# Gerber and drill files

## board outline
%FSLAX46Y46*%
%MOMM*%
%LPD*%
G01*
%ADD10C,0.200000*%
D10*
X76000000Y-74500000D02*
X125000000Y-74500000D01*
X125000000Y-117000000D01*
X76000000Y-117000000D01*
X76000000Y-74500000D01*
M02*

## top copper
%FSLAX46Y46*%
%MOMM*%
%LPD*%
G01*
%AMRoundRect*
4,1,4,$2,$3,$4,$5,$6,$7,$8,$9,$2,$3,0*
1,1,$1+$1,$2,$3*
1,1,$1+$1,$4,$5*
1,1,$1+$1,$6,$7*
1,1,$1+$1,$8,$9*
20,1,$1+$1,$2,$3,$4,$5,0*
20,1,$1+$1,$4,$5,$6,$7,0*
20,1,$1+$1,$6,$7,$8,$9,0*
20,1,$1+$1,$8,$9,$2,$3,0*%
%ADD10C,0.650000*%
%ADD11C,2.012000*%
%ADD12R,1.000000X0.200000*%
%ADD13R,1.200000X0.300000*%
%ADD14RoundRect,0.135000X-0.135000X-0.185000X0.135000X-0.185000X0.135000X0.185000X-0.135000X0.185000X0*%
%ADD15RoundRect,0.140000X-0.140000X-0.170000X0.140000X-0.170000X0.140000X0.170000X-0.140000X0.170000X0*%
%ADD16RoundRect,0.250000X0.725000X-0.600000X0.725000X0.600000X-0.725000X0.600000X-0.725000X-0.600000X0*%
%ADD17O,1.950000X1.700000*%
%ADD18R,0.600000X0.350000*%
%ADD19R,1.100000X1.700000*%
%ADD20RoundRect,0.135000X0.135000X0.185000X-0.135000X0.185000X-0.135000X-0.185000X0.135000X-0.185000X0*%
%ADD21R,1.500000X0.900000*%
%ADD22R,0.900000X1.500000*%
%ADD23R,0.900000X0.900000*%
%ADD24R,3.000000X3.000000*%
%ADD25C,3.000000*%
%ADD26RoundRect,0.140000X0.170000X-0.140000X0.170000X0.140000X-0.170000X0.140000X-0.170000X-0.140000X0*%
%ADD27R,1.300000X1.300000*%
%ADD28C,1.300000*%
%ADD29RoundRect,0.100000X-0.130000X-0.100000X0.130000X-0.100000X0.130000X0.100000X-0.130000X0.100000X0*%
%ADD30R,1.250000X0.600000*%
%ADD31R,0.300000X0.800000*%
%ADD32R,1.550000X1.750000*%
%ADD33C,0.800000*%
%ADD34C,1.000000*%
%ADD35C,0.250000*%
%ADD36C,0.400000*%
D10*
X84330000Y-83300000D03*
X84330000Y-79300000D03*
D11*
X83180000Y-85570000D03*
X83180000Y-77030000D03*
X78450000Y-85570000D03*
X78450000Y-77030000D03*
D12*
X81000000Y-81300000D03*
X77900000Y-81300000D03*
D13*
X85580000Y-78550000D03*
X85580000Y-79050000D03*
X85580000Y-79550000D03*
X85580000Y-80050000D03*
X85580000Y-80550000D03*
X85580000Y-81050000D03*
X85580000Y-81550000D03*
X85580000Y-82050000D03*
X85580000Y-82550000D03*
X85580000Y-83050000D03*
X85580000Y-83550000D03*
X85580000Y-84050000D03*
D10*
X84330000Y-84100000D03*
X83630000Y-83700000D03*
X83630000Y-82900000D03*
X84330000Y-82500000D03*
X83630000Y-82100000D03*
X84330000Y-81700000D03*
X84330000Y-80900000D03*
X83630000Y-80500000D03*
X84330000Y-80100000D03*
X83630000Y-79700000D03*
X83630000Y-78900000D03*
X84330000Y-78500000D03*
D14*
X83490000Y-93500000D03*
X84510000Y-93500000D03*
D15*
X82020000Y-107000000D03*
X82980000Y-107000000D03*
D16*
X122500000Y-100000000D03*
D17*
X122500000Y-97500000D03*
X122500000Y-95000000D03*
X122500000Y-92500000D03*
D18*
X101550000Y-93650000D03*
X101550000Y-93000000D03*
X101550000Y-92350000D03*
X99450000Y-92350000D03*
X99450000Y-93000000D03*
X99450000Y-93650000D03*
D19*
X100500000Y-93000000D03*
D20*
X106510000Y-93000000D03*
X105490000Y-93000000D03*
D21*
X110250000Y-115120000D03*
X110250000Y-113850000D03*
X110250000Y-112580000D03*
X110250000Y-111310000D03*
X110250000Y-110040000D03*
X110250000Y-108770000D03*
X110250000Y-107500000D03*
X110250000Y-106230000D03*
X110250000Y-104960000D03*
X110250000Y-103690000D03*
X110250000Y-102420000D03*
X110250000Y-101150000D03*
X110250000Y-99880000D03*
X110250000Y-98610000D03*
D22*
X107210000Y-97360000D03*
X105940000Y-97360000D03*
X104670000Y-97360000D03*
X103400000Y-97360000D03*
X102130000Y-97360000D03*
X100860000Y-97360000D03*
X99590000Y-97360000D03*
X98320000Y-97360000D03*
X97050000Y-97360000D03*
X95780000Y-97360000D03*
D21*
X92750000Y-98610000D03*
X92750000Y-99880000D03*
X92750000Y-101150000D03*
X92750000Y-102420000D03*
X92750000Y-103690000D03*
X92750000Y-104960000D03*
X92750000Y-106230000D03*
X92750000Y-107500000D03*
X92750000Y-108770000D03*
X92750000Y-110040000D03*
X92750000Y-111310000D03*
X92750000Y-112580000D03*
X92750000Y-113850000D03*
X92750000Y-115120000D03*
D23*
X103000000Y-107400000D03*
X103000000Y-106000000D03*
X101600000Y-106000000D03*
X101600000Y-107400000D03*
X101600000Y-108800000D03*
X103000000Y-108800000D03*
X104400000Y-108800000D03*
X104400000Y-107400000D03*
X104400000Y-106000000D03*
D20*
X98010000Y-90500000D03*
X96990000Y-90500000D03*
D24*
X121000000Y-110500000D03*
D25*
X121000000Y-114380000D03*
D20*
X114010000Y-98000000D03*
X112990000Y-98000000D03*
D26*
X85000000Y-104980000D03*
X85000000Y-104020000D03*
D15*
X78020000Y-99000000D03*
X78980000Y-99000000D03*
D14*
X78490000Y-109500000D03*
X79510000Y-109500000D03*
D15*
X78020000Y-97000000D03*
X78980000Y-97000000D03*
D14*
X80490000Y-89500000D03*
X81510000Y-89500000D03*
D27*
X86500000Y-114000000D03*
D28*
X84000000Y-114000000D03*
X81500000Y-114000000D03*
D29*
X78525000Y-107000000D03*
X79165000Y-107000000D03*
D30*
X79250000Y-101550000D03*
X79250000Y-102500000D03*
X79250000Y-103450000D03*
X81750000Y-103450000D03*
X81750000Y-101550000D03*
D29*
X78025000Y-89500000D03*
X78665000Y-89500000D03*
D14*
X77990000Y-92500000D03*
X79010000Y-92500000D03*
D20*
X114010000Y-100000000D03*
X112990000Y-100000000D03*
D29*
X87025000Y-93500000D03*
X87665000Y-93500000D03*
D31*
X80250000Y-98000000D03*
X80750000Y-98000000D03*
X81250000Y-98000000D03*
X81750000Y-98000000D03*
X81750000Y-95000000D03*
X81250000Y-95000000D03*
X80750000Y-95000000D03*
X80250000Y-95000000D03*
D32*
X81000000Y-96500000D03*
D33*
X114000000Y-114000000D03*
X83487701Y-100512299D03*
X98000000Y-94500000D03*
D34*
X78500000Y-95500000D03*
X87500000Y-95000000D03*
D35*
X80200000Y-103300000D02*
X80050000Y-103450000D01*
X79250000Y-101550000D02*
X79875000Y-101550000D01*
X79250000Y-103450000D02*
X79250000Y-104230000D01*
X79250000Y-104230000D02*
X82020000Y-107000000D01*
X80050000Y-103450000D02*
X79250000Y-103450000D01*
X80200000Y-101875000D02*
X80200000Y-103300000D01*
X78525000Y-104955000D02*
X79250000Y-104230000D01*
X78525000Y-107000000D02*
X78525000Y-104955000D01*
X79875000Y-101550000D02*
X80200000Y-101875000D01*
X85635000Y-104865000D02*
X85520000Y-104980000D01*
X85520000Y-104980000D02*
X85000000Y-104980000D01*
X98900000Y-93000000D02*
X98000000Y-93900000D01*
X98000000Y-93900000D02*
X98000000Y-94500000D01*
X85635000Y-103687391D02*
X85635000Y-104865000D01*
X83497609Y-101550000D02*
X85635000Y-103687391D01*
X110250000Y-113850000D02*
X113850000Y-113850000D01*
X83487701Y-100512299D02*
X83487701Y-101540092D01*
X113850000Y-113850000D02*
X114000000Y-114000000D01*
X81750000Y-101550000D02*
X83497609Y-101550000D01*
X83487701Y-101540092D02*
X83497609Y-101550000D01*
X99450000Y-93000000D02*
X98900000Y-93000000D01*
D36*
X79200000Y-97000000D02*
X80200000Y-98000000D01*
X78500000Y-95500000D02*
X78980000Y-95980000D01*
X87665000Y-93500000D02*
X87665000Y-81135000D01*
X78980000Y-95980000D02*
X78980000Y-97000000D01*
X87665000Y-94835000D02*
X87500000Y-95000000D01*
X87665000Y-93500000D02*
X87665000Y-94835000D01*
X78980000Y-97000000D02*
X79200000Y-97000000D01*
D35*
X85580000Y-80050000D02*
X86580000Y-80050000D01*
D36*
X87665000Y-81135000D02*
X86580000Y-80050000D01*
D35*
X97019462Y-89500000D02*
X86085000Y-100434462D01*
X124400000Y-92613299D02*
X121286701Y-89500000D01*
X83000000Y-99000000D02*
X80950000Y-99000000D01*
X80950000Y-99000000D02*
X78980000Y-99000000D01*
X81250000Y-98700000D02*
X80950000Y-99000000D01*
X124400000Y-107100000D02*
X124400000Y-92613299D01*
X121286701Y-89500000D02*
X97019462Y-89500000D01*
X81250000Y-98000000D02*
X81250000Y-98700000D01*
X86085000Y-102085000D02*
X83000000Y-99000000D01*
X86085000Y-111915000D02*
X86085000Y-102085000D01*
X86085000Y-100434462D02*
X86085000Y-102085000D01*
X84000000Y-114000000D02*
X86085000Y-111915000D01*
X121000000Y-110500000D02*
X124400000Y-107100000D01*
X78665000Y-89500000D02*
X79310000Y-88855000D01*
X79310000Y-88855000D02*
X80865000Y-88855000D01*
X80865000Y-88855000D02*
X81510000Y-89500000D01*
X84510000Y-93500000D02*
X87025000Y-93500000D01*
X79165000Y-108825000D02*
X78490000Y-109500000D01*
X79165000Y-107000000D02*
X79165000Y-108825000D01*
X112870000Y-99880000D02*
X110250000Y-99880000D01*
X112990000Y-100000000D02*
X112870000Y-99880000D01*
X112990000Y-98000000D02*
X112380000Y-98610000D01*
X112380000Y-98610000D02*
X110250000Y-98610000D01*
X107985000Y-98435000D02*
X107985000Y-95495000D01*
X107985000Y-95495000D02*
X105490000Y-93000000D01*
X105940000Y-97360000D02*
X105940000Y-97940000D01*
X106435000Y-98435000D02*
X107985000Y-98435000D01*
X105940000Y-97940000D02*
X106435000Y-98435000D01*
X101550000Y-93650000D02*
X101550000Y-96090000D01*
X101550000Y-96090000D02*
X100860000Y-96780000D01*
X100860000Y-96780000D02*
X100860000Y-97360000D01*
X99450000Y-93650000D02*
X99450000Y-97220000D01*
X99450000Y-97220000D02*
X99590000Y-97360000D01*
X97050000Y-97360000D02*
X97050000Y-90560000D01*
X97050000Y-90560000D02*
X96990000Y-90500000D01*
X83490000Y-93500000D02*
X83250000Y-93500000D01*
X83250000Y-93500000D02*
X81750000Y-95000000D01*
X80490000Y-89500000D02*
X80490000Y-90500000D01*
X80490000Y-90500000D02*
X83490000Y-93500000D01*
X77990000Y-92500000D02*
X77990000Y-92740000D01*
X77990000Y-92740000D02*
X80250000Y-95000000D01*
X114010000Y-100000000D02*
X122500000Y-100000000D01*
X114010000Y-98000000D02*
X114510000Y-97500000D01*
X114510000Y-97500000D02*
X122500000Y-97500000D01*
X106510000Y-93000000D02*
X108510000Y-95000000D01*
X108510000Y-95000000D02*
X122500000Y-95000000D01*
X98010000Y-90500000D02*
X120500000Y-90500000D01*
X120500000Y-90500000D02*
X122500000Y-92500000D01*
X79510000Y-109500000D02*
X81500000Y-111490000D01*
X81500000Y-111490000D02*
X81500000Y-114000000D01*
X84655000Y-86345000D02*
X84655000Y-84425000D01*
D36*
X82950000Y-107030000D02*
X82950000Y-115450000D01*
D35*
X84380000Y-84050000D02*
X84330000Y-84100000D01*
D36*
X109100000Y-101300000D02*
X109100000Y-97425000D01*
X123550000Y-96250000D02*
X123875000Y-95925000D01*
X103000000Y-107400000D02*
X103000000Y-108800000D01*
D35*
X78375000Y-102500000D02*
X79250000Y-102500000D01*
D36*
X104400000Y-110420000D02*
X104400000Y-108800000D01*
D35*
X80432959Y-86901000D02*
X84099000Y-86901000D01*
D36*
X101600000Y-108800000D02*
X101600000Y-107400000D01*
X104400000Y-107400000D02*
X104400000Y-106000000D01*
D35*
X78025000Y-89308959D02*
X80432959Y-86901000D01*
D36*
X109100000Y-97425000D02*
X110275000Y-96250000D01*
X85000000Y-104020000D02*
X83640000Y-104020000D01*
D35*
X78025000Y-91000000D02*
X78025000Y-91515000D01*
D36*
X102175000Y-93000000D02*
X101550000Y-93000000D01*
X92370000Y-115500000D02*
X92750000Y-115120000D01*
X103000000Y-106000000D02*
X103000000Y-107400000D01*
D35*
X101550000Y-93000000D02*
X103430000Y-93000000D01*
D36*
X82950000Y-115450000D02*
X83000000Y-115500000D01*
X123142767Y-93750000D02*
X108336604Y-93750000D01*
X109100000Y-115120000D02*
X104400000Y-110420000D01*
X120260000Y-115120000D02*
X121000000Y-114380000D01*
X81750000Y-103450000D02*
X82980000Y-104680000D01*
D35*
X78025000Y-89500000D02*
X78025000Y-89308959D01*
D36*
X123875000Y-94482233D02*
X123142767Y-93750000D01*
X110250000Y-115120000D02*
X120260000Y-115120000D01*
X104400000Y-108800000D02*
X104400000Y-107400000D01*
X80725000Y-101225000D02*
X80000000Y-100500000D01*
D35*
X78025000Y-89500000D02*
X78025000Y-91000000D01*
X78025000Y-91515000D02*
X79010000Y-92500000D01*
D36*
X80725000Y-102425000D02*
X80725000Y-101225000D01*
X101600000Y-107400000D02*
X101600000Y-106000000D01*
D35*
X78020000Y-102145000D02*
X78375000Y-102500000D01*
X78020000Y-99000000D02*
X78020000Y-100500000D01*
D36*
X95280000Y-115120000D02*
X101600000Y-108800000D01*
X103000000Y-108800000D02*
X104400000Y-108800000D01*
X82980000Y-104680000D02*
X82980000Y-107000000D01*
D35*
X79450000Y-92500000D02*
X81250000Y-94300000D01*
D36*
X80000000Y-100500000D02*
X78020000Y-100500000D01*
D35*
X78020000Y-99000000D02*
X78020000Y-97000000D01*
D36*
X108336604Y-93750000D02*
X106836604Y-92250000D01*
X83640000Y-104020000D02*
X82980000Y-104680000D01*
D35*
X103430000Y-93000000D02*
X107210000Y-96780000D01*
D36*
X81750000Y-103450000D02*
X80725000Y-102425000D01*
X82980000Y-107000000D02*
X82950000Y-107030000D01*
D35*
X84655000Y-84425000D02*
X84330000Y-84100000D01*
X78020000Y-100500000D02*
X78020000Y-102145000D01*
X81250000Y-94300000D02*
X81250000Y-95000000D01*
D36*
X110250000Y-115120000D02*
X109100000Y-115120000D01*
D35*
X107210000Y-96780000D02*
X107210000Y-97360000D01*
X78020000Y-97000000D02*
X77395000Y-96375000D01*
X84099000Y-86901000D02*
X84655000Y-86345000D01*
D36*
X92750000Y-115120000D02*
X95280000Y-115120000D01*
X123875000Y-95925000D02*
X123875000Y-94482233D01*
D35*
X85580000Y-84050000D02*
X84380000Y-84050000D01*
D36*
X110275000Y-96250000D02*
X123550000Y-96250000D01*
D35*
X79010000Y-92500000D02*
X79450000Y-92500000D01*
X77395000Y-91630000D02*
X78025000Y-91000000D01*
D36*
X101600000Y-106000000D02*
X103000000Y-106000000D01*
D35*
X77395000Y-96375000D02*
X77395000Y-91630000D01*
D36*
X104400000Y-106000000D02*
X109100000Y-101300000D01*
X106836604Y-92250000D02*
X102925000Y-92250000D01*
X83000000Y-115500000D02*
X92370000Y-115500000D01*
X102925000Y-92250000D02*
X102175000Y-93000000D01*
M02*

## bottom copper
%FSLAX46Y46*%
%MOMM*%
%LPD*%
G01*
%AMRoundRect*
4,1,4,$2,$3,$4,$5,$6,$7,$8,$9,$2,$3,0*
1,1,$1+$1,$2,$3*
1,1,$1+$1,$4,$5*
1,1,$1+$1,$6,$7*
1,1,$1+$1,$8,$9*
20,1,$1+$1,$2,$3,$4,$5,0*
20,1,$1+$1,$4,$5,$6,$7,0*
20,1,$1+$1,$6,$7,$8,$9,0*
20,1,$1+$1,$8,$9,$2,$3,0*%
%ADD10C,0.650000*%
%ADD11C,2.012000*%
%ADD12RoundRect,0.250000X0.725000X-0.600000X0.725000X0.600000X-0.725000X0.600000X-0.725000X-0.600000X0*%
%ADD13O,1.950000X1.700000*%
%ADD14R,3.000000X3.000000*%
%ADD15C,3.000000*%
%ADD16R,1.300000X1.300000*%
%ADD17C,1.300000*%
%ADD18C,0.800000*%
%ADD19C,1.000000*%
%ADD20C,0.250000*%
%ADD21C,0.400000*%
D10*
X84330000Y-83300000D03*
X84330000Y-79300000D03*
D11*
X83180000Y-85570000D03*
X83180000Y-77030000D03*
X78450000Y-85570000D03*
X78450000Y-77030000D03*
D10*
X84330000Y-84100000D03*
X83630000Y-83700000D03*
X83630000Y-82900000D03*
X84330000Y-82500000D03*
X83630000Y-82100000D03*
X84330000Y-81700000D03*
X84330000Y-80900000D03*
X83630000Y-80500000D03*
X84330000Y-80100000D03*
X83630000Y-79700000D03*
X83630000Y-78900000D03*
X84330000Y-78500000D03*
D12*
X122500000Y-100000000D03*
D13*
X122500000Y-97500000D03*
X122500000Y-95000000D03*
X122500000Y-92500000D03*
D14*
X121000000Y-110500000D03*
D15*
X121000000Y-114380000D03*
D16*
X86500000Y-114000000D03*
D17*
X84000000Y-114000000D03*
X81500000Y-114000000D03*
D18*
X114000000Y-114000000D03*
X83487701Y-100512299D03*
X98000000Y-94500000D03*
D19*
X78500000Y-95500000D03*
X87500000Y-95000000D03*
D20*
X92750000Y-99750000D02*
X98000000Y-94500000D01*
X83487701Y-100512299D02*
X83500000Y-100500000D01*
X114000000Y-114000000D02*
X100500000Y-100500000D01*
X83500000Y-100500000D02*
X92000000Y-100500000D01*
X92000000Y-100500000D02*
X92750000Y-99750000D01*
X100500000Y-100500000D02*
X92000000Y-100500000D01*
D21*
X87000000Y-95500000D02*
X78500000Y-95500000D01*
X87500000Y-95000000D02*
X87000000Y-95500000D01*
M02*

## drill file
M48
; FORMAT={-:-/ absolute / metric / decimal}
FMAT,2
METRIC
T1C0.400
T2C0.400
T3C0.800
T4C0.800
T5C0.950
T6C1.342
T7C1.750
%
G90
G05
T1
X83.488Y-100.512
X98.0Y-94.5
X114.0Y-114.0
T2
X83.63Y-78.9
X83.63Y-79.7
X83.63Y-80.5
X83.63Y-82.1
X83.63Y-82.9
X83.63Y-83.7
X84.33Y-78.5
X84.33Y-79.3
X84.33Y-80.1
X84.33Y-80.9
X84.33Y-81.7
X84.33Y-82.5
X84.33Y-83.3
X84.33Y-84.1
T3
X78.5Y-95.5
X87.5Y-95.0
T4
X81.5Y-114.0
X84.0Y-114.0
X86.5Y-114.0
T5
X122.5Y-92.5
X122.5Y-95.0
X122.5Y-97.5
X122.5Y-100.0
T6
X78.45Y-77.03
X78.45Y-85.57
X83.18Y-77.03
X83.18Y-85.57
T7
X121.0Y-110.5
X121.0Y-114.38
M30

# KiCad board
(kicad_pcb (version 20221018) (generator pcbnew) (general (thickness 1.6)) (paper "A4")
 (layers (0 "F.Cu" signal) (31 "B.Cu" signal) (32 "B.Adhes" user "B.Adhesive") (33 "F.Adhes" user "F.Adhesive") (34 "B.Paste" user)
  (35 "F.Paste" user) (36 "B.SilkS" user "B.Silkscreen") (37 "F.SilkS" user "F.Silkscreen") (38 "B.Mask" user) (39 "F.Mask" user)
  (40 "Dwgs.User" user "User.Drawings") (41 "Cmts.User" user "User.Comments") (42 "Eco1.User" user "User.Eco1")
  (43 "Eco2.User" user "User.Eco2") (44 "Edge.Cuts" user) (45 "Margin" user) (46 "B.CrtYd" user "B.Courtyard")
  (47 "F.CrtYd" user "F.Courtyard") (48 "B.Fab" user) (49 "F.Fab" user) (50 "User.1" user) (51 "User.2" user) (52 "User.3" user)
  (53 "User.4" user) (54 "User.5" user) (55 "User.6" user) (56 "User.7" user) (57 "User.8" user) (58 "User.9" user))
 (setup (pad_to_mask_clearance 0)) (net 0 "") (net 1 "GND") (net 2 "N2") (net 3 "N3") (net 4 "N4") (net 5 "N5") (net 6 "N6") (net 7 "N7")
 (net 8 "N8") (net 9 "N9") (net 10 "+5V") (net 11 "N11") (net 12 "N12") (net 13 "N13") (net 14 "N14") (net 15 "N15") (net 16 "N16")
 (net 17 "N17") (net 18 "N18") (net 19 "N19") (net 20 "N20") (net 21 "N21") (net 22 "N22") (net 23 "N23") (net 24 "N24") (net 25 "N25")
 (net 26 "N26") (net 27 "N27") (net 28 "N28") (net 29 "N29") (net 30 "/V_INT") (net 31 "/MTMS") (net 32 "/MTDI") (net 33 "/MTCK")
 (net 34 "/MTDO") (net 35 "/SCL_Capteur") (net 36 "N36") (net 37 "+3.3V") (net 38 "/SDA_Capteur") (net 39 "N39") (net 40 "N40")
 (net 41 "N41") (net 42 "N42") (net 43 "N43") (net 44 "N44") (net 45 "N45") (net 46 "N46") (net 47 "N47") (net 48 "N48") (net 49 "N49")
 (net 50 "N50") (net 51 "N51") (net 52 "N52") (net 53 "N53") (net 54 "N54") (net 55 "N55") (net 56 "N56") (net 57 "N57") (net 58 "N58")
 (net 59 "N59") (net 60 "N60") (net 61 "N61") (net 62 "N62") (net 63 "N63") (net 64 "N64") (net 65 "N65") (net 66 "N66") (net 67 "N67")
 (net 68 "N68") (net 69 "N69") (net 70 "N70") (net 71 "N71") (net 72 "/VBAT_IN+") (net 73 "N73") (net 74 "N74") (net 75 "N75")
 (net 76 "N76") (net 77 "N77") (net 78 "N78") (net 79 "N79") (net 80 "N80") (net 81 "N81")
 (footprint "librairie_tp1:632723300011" (layer "F.Cu") (at 79.685 81.3 -90)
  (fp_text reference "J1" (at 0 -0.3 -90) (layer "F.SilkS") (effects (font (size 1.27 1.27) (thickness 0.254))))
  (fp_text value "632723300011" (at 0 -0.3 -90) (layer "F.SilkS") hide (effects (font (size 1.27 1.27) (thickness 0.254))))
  (pad "1" thru_hole circle (at 2 -4.645 270) (size 0.65 0.65) (drill 0.4) (layers "*.Cu" "*.Mask") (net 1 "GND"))
  (pad "2" thru_hole circle (at -2 -4.645 270) (size 0.65 0.65) (drill 0.4) (layers "*.Cu" "*.Mask") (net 1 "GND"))
  (pad "3" thru_hole circle (at 4.27 -3.495 270) (size 2.012 2.012) (drill 1.3416) (layers "*.Cu" "*.Mask") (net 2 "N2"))
  (pad "4" thru_hole circle (at -4.27 -3.495 270) (size 2.012 2.012) (drill 1.3416) (layers "*.Cu" "*.Mask") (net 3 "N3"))
  (pad "5" thru_hole circle (at 4.27 1.235 270) (size 2.012 2.012) (drill 1.3416) (layers "*.Cu" "*.Mask") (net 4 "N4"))
  (pad "6" thru_hole circle (at -4.27 1.235 270) (size 2.012 2.012) (drill 1.3416) (layers "*.Cu" "*.Mask") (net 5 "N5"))
  (pad "7" smd rect (at 0 -1.315 270) (size 0.2 1) (layers "F.Cu" "F.Paste" "F.Mask") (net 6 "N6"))
  (pad "8" smd rect (at 0 1.785 270) (size 0.2 1) (layers "F.Cu" "F.Paste" "F.Mask") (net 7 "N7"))
  (pad "A1" smd rect (at -2.75 -5.895 270) (size 0.3 1.2) (layers "F.Cu" "F.Paste" "F.Mask") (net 1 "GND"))
  (pad "A2" smd rect (at -2.25 -5.895 270) (size 0.3 1.2) (layers "F.Cu" "F.Paste" "F.Mask") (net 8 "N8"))
  (pad "A3" smd rect (at -1.75 -5.895 270) (size 0.3 1.2) (layers "F.Cu" "F.Paste" "F.Mask") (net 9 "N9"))
  (pad "A4" smd rect (at -1.25 -5.895 270) (size 0.3 1.2) (layers "F.Cu" "F.Paste" "F.Mask") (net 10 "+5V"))
  (pad "A5" smd rect (at -0.75 -5.895 270) (size 0.3 1.2) (layers "F.Cu" "F.Paste" "F.Mask") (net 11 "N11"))
  (pad "A6" smd rect (at -0.25 -5.895 270) (size 0.3 1.2) (layers "F.Cu" "F.Paste" "F.Mask") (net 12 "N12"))
  (pad "A7" smd rect (at 0.25 -5.895 270) (size 0.3 1.2) (layers "F.Cu" "F.Paste" "F.Mask") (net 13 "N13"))
  (pad "A8" smd rect (at 0.75 -5.895 270) (size 0.3 1.2) (layers "F.Cu" "F.Paste" "F.Mask") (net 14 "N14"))
  (pad "A9" smd rect (at 1.25 -5.895 270) (size 0.3 1.2) (layers "F.Cu" "F.Paste" "F.Mask") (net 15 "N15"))
  (pad "A10" smd rect (at 1.75 -5.895 270) (size 0.3 1.2) (layers "F.Cu" "F.Paste" "F.Mask") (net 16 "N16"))
  (pad "A11" smd rect (at 2.25 -5.895 270) (size 0.3 1.2) (layers "F.Cu" "F.Paste" "F.Mask") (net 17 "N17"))
  (pad "A12" smd rect (at 2.75 -5.895 270) (size 0.3 1.2) (layers "F.Cu" "F.Paste" "F.Mask") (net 1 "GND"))
  (pad "B1" thru_hole circle (at 2.8 -4.645 270) (size 0.65 0.65) (drill 0.4) (layers "*.Cu" "*.Mask") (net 1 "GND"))
  (pad "B2" thru_hole circle (at 2.4 -3.945 270) (size 0.65 0.65) (drill 0.4) (layers "*.Cu" "*.Mask") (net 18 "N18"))
  (pad "B3" thru_hole circle (at 1.6 -3.945 270) (size 0.65 0.65) (drill 0.4) (layers "*.Cu" "*.Mask") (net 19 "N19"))
  (pad "B4" thru_hole circle (at 1.2 -4.645 270) (size 0.65 0.65) (drill 0.4) (layers "*.Cu" "*.Mask") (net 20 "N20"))
  (pad "B5" thru_hole circle (at 0.8 -3.945 270) (size 0.65 0.65) (drill 0.4) (layers "*.Cu" "*.Mask") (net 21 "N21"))
  (pad "B6" thru_hole circle (at 0.4 -4.645 270) (size 0.65 0.65) (drill 0.4) (layers "*.Cu" "*.Mask") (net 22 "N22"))
  (pad "B7" thru_hole circle (at -0.4 -4.645 270) (size 0.65 0.65) (drill 0.4) (layers "*.Cu" "*.Mask") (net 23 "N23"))
  (pad "B8" thru_hole circle (at -0.8 -3.945 270) (size 0.65 0.65) (drill 0.4) (layers "*.Cu" "*.Mask") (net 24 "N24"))
  (pad "B9" thru_hole circle (at -1.2 -4.645 270) (size 0.65 0.65) (drill 0.4) (layers "*.Cu" "*.Mask") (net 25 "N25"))
  (pad "B10" thru_hole circle (at -1.6 -3.945 270) (size 0.65 0.65) (drill 0.4) (layers "*.Cu" "*.Mask") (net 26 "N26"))
  (pad "B11" thru_hole circle (at -2.4 -3.945 270) (size 0.65 0.65) (drill 0.4) (layers "*.Cu" "*.Mask") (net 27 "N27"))
  (pad "B12" thru_hole circle (at -2.8 -4.645 270) (size 0.65 0.65) (drill 0.4) (layers "*.Cu" "*.Mask") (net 1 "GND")))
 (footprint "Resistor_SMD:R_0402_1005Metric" (layer "F.Cu") (at 84 93.5)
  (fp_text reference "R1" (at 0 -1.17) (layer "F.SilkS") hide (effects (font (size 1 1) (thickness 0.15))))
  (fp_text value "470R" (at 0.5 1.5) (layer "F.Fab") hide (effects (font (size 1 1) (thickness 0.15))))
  (pad "1" smd roundrect (at -0.51 0) (size 0.54 0.64) (layers "F.Cu" "F.Paste" "F.Mask") (roundrect_rratio 0.25) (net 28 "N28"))
  (pad "2" smd roundrect (at 0.51 0) (size 0.54 0.64) (layers "F.Cu" "F.Paste" "F.Mask") (roundrect_rratio 0.25) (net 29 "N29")))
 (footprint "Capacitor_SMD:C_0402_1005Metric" (layer "F.Cu") (at 82.5 107)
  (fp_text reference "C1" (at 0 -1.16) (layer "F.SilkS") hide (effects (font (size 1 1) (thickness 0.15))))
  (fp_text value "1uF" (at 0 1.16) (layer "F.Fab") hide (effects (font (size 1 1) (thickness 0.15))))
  (pad "1" smd roundrect (at -0.48 0) (size 0.56 0.62) (layers "F.Cu" "F.Paste" "F.Mask") (roundrect_rratio 0.25) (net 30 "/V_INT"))
  (pad "2" smd roundrect (at 0.48 0) (size 0.56 0.62) (layers "F.Cu" "F.Paste" "F.Mask") (roundrect_rratio 0.25) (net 1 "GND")))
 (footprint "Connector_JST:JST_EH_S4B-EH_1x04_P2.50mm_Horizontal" (layer "F.Cu") (at 122.5 100 90)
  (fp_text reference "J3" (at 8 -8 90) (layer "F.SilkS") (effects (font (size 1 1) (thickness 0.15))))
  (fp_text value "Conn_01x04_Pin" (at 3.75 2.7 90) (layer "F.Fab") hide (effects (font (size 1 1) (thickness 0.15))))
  (pad "1" thru_hole roundrect (at 0 0 90) (size 1.7 1.95) (drill 0.95) (layers "*.Cu" "*.Mask") (roundrect_rratio 0.147059)
   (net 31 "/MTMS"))
  (pad "2" thru_hole oval (at 2.5 0 90) (size 1.7 1.95) (drill 0.95) (layers "*.Cu" "*.Mask") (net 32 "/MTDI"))
  (pad "3" thru_hole oval (at 5 0 90) (size 1.7 1.95) (drill 0.95) (layers "*.Cu" "*.Mask") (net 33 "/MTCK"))
  (pad "4" thru_hole oval (at 7.5 0 90) (size 1.7 1.95) (drill 0.95) (layers "*.Cu" "*.Mask") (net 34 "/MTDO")))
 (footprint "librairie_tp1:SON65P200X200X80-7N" (layer "F.Cu") (at 100.5 93 180)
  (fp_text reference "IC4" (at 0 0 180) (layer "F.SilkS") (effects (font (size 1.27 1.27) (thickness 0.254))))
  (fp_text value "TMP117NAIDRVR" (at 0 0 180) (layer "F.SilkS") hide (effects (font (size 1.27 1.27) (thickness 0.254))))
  (pad "1" smd rect (at -1.05 -0.65 270) (size 0.35 0.6) (layers "F.Cu" "F.Paste" "F.Mask") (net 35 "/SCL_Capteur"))
  (pad "2" smd rect (at -1.05 0 270) (size 0.35 0.6) (layers "F.Cu" "F.Paste" "F.Mask") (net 1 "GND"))
  (pad "3" smd rect (at -1.05 0.65 270) (size 0.35 0.6) (layers "F.Cu" "F.Paste" "F.Mask") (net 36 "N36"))
  (pad "4" smd rect (at 1.05 0.65 270) (size 0.35 0.6) (layers "F.Cu" "F.Paste" "F.Mask") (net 1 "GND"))
  (pad "5" smd rect (at 1.05 0 270) (size 0.35 0.6) (layers "F.Cu" "F.Paste" "F.Mask") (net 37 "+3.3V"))
  (pad "6" smd rect (at 1.05 -0.65 270) (size 0.35 0.6) (layers "F.Cu" "F.Paste" "F.Mask") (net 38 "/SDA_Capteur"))
  (pad "7" smd rect (at 0 0 180) (size 1.1 1.7) (layers "F.Cu" "F.Paste" "F.Mask") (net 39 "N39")))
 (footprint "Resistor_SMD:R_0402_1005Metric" (layer "F.Cu") (at 106 93 180)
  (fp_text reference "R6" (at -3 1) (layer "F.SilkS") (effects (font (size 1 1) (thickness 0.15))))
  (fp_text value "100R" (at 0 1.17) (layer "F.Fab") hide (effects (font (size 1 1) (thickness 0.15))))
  (pad "1" smd roundrect (at -0.51 0 180) (size 0.54 0.64) (layers "F.Cu" "F.Paste" "F.Mask") (roundrect_rratio 0.25) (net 33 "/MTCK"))
  (pad "2" smd roundrect (at 0.51 0 180) (size 0.54 0.64) (layers "F.Cu" "F.Paste" "F.Mask") (roundrect_rratio 0.25) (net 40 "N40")))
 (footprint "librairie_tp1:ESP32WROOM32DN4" (layer "F.Cu") (at 101.5 109.86 180)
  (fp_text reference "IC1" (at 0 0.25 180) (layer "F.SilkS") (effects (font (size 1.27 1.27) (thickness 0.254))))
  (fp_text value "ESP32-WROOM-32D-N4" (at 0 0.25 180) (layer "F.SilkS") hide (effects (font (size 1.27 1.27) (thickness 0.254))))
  (pad "1" smd rect (at -8.75 -5.26 270) (size 0.9 1.5) (layers "F.Cu" "F.Paste" "F.Mask") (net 1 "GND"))
  (pad "2" smd rect (at -8.75 -3.99 270) (size 0.9 1.5) (layers "F.Cu" "F.Paste" "F.Mask") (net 37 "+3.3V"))
  (pad "3" smd rect (at -8.75 -2.72 270) (size 0.9 1.5) (layers "F.Cu" "F.Paste" "F.Mask") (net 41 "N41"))
  (pad "4" smd rect (at -8.75 -1.45 270) (size 0.9 1.5) (layers "F.Cu" "F.Paste" "F.Mask") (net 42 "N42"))
  (pad "5" smd rect (at -8.75 -0.18 270) (size 0.9 1.5) (layers "F.Cu" "F.Paste" "F.Mask") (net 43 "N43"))
  (pad "6" smd rect (at -8.75 1.09 270) (size 0.9 1.5) (layers "F.Cu" "F.Paste" "F.Mask") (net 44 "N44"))
  (pad "7" smd rect (at -8.75 2.36 270) (size 0.9 1.5) (layers "F.Cu" "F.Paste" "F.Mask") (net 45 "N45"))
  (pad "8" smd rect (at -8.75 3.63 270) (size 0.9 1.5) (layers "F.Cu" "F.Paste" "F.Mask") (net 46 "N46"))
  (pad "9" smd rect (at -8.75 4.9 270) (size 0.9 1.5) (layers "F.Cu" "F.Paste" "F.Mask") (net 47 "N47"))
  (pad "10" smd rect (at -8.75 6.17 270) (size 0.9 1.5) (layers "F.Cu" "F.Paste" "F.Mask") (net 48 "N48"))
  (pad "11" smd rect (at -8.75 7.44 270) (size 0.9 1.5) (layers "F.Cu" "F.Paste" "F.Mask") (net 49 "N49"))
  (pad "12" smd rect (at -8.75 8.71 270) (size 0.9 1.5) (layers "F.Cu" "F.Paste" "F.Mask") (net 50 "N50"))
  (pad "13" smd rect (at -8.75 9.98 270) (size 0.9 1.5) (layers "F.Cu" "F.Paste" "F.Mask") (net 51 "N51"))
  (pad "14" smd rect (at -8.75 11.25 270) (size 0.9 1.5) (layers "F.Cu" "F.Paste" "F.Mask") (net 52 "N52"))
  (pad "15" smd rect (at -5.71 12.5 180) (size 0.9 1.5) (layers "F.Cu" "F.Paste" "F.Mask") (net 1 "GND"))
  (pad "16" smd rect (at -4.44 12.5 180) (size 0.9 1.5) (layers "F.Cu" "F.Paste" "F.Mask") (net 40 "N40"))
  (pad "17" smd rect (at -3.17 12.5 180) (size 0.9 1.5) (layers "F.Cu" "F.Paste" "F.Mask") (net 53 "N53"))
  (pad "18" smd rect (at -1.9 12.5 180) (size 0.9 1.5) (layers "F.Cu" "F.Paste" "F.Mask") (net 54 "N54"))
  (pad "19" smd rect (at -0.63 12.5 180) (size 0.9 1.5) (layers "F.Cu" "F.Paste" "F.Mask") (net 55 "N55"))
  (pad "20" smd rect (at 0.64 12.5 180) (size 0.9 1.5) (layers "F.Cu" "F.Paste" "F.Mask") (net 35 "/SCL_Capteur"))
  (pad "21" smd rect (at 1.91 12.5 180) (size 0.9 1.5) (layers "F.Cu" "F.Paste" "F.Mask") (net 38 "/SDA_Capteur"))
  (pad "22" smd rect (at 3.18 12.5 180) (size 0.9 1.5) (layers "F.Cu" "F.Paste" "F.Mask") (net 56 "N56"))
  (pad "23" smd rect (at 4.45 12.5 180) (size 0.9 1.5) (layers "F.Cu" "F.Paste" "F.Mask") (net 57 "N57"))
  (pad "24" smd rect (at 5.72 12.5 180) (size 0.9 1.5) (layers "F.Cu" "F.Paste" "F.Mask") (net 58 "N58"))
  (pad "25" smd rect (at 8.75 11.25 270) (size 0.9 1.5) (layers "F.Cu" "F.Paste" "F.Mask") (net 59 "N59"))
  (pad "26" smd rect (at 8.75 9.98 270) (size 0.9 1.5) (layers "F.Cu" "F.Paste" "F.Mask") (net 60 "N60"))
  (pad "27" smd rect (at 8.75 8.71 270) (size 0.9 1.5) (layers "F.Cu" "F.Paste" "F.Mask") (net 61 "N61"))
  (pad "28" smd rect (at 8.75 7.44 270) (size 0.9 1.5) (layers "F.Cu" "F.Paste" "F.Mask") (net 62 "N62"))
  (pad "29" smd rect (at 8.75 6.17 270) (size 0.9 1.5) (layers "F.Cu" "F.Paste" "F.Mask") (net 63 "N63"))
  (pad "30" smd rect (at 8.75 4.9 270) (size 0.9 1.5) (layers "F.Cu" "F.Paste" "F.Mask") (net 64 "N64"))
  (pad "31" smd rect (at 8.75 3.63 270) (size 0.9 1.5) (layers "F.Cu" "F.Paste" "F.Mask") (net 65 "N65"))
  (pad "32" smd rect (at 8.75 2.36 270) (size 0.9 1.5) (layers "F.Cu" "F.Paste" "F.Mask") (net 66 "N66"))
  (pad "33" smd rect (at 8.75 1.09 270) (size 0.9 1.5) (layers "F.Cu" "F.Paste" "F.Mask") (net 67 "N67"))
  (pad "34" smd rect (at 8.75 -0.18 270) (size 0.9 1.5) (layers "F.Cu" "F.Paste" "F.Mask") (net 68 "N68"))
  (pad "35" smd rect (at 8.75 -1.45 270) (size 0.9 1.5) (layers "F.Cu" "F.Paste" "F.Mask") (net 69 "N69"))
  (pad "36" smd rect (at 8.75 -2.72 270) (size 0.9 1.5) (layers "F.Cu" "F.Paste" "F.Mask") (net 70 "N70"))
  (pad "37" smd rect (at 8.75 -3.99 270) (size 0.9 1.5) (layers "F.Cu" "F.Paste" "F.Mask") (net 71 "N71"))
  (pad "38" smd rect (at 8.75 -5.26 270) (size 0.9 1.5) (layers "F.Cu" "F.Paste" "F.Mask") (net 1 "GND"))
  (pad "39" smd rect (at -1.5 2.46 180) (size 0.9 0.9) (layers "F.Cu" "F.Paste" "F.Mask") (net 1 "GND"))
  (pad "40" smd rect (at -1.5 3.86 180) (size 0.9 0.9) (layers "F.Cu" "F.Paste" "F.Mask") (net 1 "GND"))
  (pad "41" smd rect (at -0.1 3.86 180) (size 0.9 0.9) (layers "F.Cu" "F.Paste" "F.Mask") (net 1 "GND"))
  (pad "42" smd rect (at -0.1 2.46 180) (size 0.9 0.9) (layers "F.Cu" "F.Paste" "F.Mask") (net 1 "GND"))
  (pad "43" smd rect (at -0.1 1.06 180) (size 0.9 0.9) (layers "F.Cu" "F.Paste" "F.Mask") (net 1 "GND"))
  (pad "44" smd rect (at -1.5 1.06 180) (size 0.9 0.9) (layers "F.Cu" "F.Paste" "F.Mask") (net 1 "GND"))
  (pad "45" smd rect (at -2.9 1.06 180) (size 0.9 0.9) (layers "F.Cu" "F.Paste" "F.Mask") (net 1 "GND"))
  (pad "46" smd rect (at -2.9 2.46 180) (size 0.9 0.9) (layers "F.Cu" "F.Paste" "F.Mask") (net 1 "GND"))
  (pad "47" smd rect (at -2.9 3.86 180) (size 0.9 0.9) (layers "F.Cu" "F.Paste" "F.Mask") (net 1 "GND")))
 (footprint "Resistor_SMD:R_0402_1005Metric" (layer "F.Cu") (at 97.5 90.5 180)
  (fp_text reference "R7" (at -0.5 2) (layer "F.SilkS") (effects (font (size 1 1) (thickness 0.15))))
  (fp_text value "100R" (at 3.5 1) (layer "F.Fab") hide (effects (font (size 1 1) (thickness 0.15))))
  (pad "1" smd roundrect (at -0.51 0 180) (size 0.54 0.64) (layers "F.Cu" "F.Paste" "F.Mask") (roundrect_rratio 0.25) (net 34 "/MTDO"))
  (pad "2" smd roundrect (at 0.51 0 180) (size 0.54 0.64) (layers "F.Cu" "F.Paste" "F.Mask") (roundrect_rratio 0.25) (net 57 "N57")))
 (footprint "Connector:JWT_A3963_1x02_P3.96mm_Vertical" (layer "F.Cu") (at 121 110.5 -90)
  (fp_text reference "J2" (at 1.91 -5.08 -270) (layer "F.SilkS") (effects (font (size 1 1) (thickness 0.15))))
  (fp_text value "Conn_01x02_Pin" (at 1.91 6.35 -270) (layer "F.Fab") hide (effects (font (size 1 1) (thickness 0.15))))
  (pad "1" thru_hole rect (at 0 0 270) (size 3 3) (drill 1.75) (layers "*.Cu" "*.Mask") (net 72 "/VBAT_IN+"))
  (pad "2" thru_hole circle (at 3.88 0 270) (size 3 3) (drill 1.75) (layers "*.Cu" "*.Mask") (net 1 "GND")))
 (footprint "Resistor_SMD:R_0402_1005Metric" (layer "F.Cu") (at 113.5 98 180)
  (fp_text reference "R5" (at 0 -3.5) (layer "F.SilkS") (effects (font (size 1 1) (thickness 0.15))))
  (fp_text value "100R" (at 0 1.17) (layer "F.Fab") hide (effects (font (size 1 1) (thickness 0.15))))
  (pad "1" smd roundrect (at -0.51 0 180) (size 0.54 0.64) (layers "F.Cu" "F.Paste" "F.Mask") (roundrect_rratio 0.25) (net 32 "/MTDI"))
  (pad "2" smd roundrect (at 0.51 0 180) (size 0.54 0.64) (layers "F.Cu" "F.Paste" "F.Mask") (roundrect_rratio 0.25) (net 52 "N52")))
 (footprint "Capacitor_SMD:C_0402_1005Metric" (layer "F.Cu") (at 85 104.5 90)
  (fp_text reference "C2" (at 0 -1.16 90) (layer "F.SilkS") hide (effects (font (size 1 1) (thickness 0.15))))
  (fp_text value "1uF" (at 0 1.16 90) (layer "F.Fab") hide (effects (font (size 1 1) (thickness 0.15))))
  (pad "1" smd roundrect (at -0.48 0 90) (size 0.56 0.62) (layers "F.Cu" "F.Paste" "F.Mask") (roundrect_rratio 0.25) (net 37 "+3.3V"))
  (pad "2" smd roundrect (at 0.48 0 90) (size 0.56 0.62) (layers "F.Cu" "F.Paste" "F.Mask") (roundrect_rratio 0.25) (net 1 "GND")))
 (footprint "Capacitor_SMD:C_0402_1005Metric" (layer "F.Cu") (at 78.5 99)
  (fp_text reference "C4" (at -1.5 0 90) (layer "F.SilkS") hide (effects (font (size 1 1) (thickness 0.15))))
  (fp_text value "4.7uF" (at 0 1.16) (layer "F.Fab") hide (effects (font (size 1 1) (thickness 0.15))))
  (pad "1" smd roundrect (at -0.48 0) (size 0.56 0.62) (layers "F.Cu" "F.Paste" "F.Mask") (roundrect_rratio 0.25) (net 1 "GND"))
  (pad "2" smd roundrect (at 0.48 0) (size 0.56 0.62) (layers "F.Cu" "F.Paste" "F.Mask") (roundrect_rratio 0.25) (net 72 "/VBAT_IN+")))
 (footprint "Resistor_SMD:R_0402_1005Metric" (layer "F.Cu") (at 79 109.5)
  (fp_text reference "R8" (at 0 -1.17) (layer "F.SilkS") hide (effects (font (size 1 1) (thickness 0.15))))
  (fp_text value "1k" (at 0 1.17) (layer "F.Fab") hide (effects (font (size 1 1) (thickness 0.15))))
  (pad "1" smd roundrect (at -0.51 0) (size 0.54 0.64) (layers "F.Cu" "F.Paste" "F.Mask") (roundrect_rratio 0.25) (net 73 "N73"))
  (pad "2" smd roundrect (at 0.51 0) (size 0.54 0.64) (layers "F.Cu" "F.Paste" "F.Mask") (roundrect_rratio 0.25) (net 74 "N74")))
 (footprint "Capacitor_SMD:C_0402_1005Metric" (layer "F.Cu") (at 78.5 97)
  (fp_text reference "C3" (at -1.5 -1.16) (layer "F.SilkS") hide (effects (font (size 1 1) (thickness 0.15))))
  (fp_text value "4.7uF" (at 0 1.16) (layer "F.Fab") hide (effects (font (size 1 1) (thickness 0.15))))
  (pad "1" smd roundrect (at -0.48 0) (size 0.56 0.62) (layers "F.Cu" "F.Paste" "F.Mask") (roundrect_rratio 0.25) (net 1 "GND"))
  (pad "2" smd roundrect (at 0.48 0) (size 0.56 0.62) (layers "F.Cu" "F.Paste" "F.Mask") (roundrect_rratio 0.25) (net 10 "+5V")))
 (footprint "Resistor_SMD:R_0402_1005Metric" (layer "F.Cu") (at 81 89.5)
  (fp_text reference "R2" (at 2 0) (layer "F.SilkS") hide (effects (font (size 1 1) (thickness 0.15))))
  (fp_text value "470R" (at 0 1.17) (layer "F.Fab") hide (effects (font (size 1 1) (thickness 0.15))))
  (pad "1" smd roundrect (at -0.51 0) (size 0.54 0.64) (layers "F.Cu" "F.Paste" "F.Mask") (roundrect_rratio 0.25) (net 28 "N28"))
  (pad "2" smd roundrect (at 0.51 0) (size 0.54 0.64) (layers "F.Cu" "F.Paste" "F.Mask") (roundrect_rratio 0.25) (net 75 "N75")))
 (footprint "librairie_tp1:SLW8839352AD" (layer "F.Cu") (at 86.5 114 180)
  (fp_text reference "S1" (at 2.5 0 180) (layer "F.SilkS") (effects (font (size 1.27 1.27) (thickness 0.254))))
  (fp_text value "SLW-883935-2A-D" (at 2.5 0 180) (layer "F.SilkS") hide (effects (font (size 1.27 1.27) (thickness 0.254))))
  (pad "1" thru_hole rect (at 0 0 180) (size 1.3 1.3) (drill 0.8) (layers "*.Cu" "*.Mask") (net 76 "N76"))
  (pad "2" thru_hole circle (at 2.5 0 180) (size 1.3 1.3) (drill 0.8) (layers "*.Cu" "*.Mask") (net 72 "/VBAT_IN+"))
  (pad "3" thru_hole circle (at 5 0 180) (size 1.3 1.3) (drill 0.8) (layers "*.Cu" "*.Mask") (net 74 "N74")))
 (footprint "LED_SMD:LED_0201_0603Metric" (layer "F.Cu") (at 78.845 107)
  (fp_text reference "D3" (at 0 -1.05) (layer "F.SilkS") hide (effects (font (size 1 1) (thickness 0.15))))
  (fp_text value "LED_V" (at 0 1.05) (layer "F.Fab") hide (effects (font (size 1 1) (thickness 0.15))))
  (pad "" smd roundrect (at -0.345 0) (size 0.318 0.36) (layers "F.Paste") (roundrect_rratio 0.25))
  (pad "" smd roundrect (at 0.345 0) (size 0.318 0.36) (layers "F.Paste") (roundrect_rratio 0.25))
  (pad "1" smd roundrect (at -0.32 0) (size 0.46 0.4) (layers "F.Cu" "F.Mask") (roundrect_rratio 0.25) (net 30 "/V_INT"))
  (pad "2" smd roundrect (at 0.32 0) (size 0.46 0.4) (layers "F.Cu" "F.Mask") (roundrect_rratio 0.25) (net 73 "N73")))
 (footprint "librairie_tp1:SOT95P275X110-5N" (layer "F.Cu") (at 80.5 102.5)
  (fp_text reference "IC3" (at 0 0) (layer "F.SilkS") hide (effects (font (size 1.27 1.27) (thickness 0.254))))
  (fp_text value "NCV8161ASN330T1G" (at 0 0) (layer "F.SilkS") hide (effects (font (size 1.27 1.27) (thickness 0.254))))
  (pad "1" smd rect (at -1.25 -0.95 90) (size 0.6 1.25) (layers "F.Cu" "F.Paste" "F.Mask") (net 30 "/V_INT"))
  (pad "2" smd rect (at -1.25 0 90) (size 0.6 1.25) (layers "F.Cu" "F.Paste" "F.Mask") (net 1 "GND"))
  (pad "3" smd rect (at -1.25 0.95 90) (size 0.6 1.25) (layers "F.Cu" "F.Paste" "F.Mask") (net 30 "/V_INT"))
  (pad "4" smd rect (at 1.25 0.95 90) (size 0.6 1.25) (layers "F.Cu" "F.Paste" "F.Mask") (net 1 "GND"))
  (pad "5" smd rect (at 1.25 -0.95 90) (size 0.6 1.25) (layers "F.Cu" "F.Paste" "F.Mask") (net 37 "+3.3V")))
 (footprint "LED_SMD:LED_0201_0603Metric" (layer "F.Cu") (at 78.345 89.5)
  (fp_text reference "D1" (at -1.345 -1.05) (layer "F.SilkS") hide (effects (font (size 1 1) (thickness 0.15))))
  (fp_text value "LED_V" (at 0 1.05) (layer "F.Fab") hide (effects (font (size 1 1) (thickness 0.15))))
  (pad "" smd roundrect (at -0.345 0) (size 0.318 0.36) (layers "F.Paste") (roundrect_rratio 0.25))
  (pad "" smd roundrect (at 0.345 0) (size 0.318 0.36) (layers "F.Paste") (roundrect_rratio 0.25))
  (pad "1" smd roundrect (at -0.32 0) (size 0.46 0.4) (layers "F.Cu" "F.Mask") (roundrect_rratio 0.25) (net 1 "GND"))
  (pad "2" smd roundrect (at 0.32 0) (size 0.46 0.4) (layers "F.Cu" "F.Mask") (roundrect_rratio 0.25) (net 75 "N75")))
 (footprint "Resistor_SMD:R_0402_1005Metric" (layer "F.Cu") (at 78.5 92.5)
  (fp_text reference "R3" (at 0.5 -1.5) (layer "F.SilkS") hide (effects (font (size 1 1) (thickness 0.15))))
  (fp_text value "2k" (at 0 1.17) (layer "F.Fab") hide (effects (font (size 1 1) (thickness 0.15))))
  (pad "1" smd roundrect (at -0.51 0) (size 0.54 0.64) (layers "F.Cu" "F.Paste" "F.Mask") (roundrect_rratio 0.25) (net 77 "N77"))
  (pad "2" smd roundrect (at 0.51 0) (size 0.54 0.64) (layers "F.Cu" "F.Paste" "F.Mask") (roundrect_rratio 0.25) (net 1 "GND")))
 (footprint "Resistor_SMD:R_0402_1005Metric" (layer "F.Cu") (at 113.5 100 180)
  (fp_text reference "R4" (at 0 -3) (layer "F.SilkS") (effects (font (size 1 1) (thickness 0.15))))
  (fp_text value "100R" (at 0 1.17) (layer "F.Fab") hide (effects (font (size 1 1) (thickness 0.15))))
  (pad "1" smd roundrect (at -0.51 0 180) (size 0.54 0.64) (layers "F.Cu" "F.Paste" "F.Mask") (roundrect_rratio 0.25) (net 31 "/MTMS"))
  (pad "2" smd roundrect (at 0.51 0 180) (size 0.54 0.64) (layers "F.Cu" "F.Paste" "F.Mask") (roundrect_rratio 0.25) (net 51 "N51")))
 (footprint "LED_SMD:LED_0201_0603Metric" (layer "F.Cu") (at 87.345 93.5)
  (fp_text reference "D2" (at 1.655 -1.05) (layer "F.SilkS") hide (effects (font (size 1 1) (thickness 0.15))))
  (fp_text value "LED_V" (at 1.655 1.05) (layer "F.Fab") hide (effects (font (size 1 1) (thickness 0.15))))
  (pad "" smd roundrect (at -0.345 0) (size 0.318 0.36) (layers "F.Paste") (roundrect_rratio 0.25))
  (pad "" smd roundrect (at 0.345 0) (size 0.318 0.36) (layers "F.Paste") (roundrect_rratio 0.25))
  (pad "1" smd roundrect (at -0.32 0) (size 0.46 0.4) (layers "F.Cu" "F.Mask") (roundrect_rratio 0.25) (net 29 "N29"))
  (pad "2" smd roundrect (at 0.32 0) (size 0.46 0.4) (layers "F.Cu" "F.Mask") (roundrect_rratio 0.25) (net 10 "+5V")))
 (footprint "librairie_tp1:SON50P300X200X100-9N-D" (layer "F.Cu") (at 81 96.5 90)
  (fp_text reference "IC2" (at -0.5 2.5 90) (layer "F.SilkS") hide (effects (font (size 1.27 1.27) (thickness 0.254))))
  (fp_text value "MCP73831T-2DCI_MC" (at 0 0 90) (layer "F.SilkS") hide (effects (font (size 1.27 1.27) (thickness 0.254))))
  (pad "1" smd rect (at -1.5 -0.75 180) (size 0.3 0.8) (layers "F.Cu" "F.Paste" "F.Mask") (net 10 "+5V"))
  (pad "2" smd rect (at -1.5 -0.25 180) (size 0.3 0.8) (layers "F.Cu" "F.Paste" "F.Mask") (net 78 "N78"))
  (pad "3" smd rect (at -1.5 0.25 180) (size 0.3 0.8) (layers "F.Cu" "F.Paste" "F.Mask") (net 72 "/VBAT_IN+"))
  (pad "4" smd rect (at -1.5 0.75 180) (size 0.3 0.8) (layers "F.Cu" "F.Paste" "F.Mask") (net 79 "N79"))
  (pad "5" smd rect (at 1.5 0.75 180) (size 0.3 0.8) (layers "F.Cu" "F.Paste" "F.Mask") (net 28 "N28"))
  (pad "6" smd rect (at 1.5 0.25 180) (size 0.3 0.8) (layers "F.Cu" "F.Paste" "F.Mask") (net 1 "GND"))
  (pad "7" smd rect (at 1.5 -0.25 180) (size 0.3 0.8) (layers "F.Cu" "F.Paste" "F.Mask") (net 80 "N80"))
  (pad "8" smd rect (at 1.5 -0.75 180) (size 0.3 0.8) (layers "F.Cu" "F.Paste" "F.Mask") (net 77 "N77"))
  (pad "9" smd rect (at 0 0 180) (size 1.55 1.75) (layers "F.Cu" "F.Paste" "F.Mask") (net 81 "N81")))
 (gr_rect (start 76 74.5) (end 125 117) (stroke (width 0.2) (type default)) (fill none) (layer "Edge.Cuts"))
 (segment (start 80.2 103.3) (end 80.05 103.45) (width 0.25) (layer "F.Cu") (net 30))
 (segment (start 79.25 101.55) (end 79.875 101.55) (width 0.25) (layer "F.Cu") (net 30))
 (segment (start 79.25 103.45) (end 79.25 104.23) (width 0.25) (layer "F.Cu") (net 30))
 (segment (start 79.25 104.23) (end 82.02 107) (width 0.25) (layer "F.Cu") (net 30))
 (segment (start 80.05 103.45) (end 79.25 103.45) (width 0.25) (layer "F.Cu") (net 30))
 (segment (start 80.2 101.875) (end 80.2 103.3) (width 0.25) (layer "F.Cu") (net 30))
 (segment (start 78.525 104.955) (end 79.25 104.23) (width 0.25) (layer "F.Cu") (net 30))
 (segment (start 78.525 107) (end 78.525 104.955) (width 0.25) (layer "F.Cu") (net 30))
 (segment (start 79.875 101.55) (end 80.2 101.875) (width 0.25) (layer "F.Cu") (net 30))
 (segment (start 85.635 104.865) (end 85.52 104.98) (width 0.25) (layer "F.Cu") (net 37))
 (segment (start 85.52 104.98) (end 85 104.98) (width 0.25) (layer "F.Cu") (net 37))
 (segment (start 98.9 93) (end 98 93.9) (width 0.25) (layer "F.Cu") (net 37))
 (segment (start 98 93.9) (end 98 94.5) (width 0.25) (layer "F.Cu") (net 37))
 (segment (start 85.635 103.687391) (end 85.635 104.865) (width 0.25) (layer "F.Cu") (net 37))
 (segment (start 83.497609 101.55) (end 85.635 103.687391) (width 0.25) (layer "F.Cu") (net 37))
 (segment (start 110.25 113.85) (end 113.85 113.85) (width 0.25) (layer "F.Cu") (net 37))
 (segment (start 83.487701 100.512299) (end 83.487701 101.540092) (width 0.25) (layer "F.Cu") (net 37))
 (segment (start 113.85 113.85) (end 114 114) (width 0.25) (layer "F.Cu") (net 37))
 (segment (start 81.75 101.55) (end 83.497609 101.55) (width 0.25) (layer "F.Cu") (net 37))
 (segment (start 83.487701 101.540092) (end 83.497609 101.55) (width 0.25) (layer "F.Cu") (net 37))
 (segment (start 99.45 93) (end 98.9 93) (width 0.25) (layer "F.Cu") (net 37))
 (via (at 114 114) (size 0.8) (drill 0.4) (layers "F.Cu" "B.Cu") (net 37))
 (via (at 83.487701 100.512299) (size 0.8) (drill 0.4) (layers "F.Cu" "B.Cu") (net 37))
 (via (at 98 94.5) (size 0.8) (drill 0.4) (layers "F.Cu" "B.Cu") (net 37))
 (segment (start 92.75 99.75) (end 98 94.5) (width 0.25) (layer "B.Cu") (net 37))
 (segment (start 83.487701 100.512299) (end 83.5 100.5) (width 0.25) (layer "B.Cu") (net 37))
 (segment (start 114 114) (end 100.5 100.5) (width 0.25) (layer "B.Cu") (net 37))
 (segment (start 83.5 100.5) (end 92 100.5) (width 0.25) (layer "B.Cu") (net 37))
 (segment (start 92 100.5) (end 92.75 99.75) (width 0.25) (layer "B.Cu") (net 37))
 (segment (start 100.5 100.5) (end 92 100.5) (width 0.25) (layer "B.Cu") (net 37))
 (segment (start 79.2 97) (end 80.2 98) (width 0.4) (layer "F.Cu") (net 10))
 (segment (start 78.5 95.5) (end 78.98 95.98) (width 0.4) (layer "F.Cu") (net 10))
 (segment (start 87.665 93.5) (end 87.665 81.135) (width 0.4) (layer "F.Cu") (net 10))
 (segment (start 78.98 95.98) (end 78.98 97) (width 0.4) (layer "F.Cu") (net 10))
 (segment (start 87.665 94.835) (end 87.5 95) (width 0.4) (layer "F.Cu") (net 10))
 (segment (start 87.665 93.5) (end 87.665 94.835) (width 0.4) (layer "F.Cu") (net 10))
 (segment (start 78.98 97) (end 79.2 97) (width 0.4) (layer "F.Cu") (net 10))
 (segment (start 85.58 80.05) (end 86.58 80.05) (width 0.25) (layer "F.Cu") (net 10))
 (segment (start 87.665 81.135) (end 86.58 80.05) (width 0.4) (layer "F.Cu") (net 10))
 (via (at 78.5 95.5) (size 1) (drill 0.8) (layers "F.Cu" "B.Cu") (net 10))
 (via (at 87.5 95) (size 1) (drill 0.8) (layers "F.Cu" "B.Cu") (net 10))
 (segment (start 87 95.5) (end 78.5 95.5) (width 0.4) (layer "B.Cu") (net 10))
 (segment (start 87.5 95) (end 87 95.5) (width 0.4) (layer "B.Cu") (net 10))
 (segment (start 97.019462 89.5) (end 86.085 100.434462) (width 0.25) (layer "F.Cu") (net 72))
 (segment (start 124.4 92.613299) (end 121.286701 89.5) (width 0.25) (layer "F.Cu") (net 72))
 (segment (start 83 99) (end 80.95 99) (width 0.25) (layer "F.Cu") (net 72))
 (segment (start 80.95 99) (end 78.98 99) (width 0.25) (layer "F.Cu") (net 72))
 (segment (start 81.25 98.7) (end 80.95 99) (width 0.25) (layer "F.Cu") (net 72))
 (segment (start 124.4 107.1) (end 124.4 92.613299) (width 0.25) (layer "F.Cu") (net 72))
 (segment (start 121.286701 89.5) (end 97.019462 89.5) (width 0.25) (layer "F.Cu") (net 72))
 (segment (start 81.25 98) (end 81.25 98.7) (width 0.25) (layer "F.Cu") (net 72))
 (segment (start 86.085 102.085) (end 83 99) (width 0.25) (layer "F.Cu") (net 72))
 (segment (start 86.085 111.915) (end 86.085 102.085) (width 0.25) (layer "F.Cu") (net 72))
 (segment (start 86.085 100.434462) (end 86.085 102.085) (width 0.25) (layer "F.Cu") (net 72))
 (segment (start 84 114) (end 86.085 111.915) (width 0.25) (layer "F.Cu") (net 72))
 (segment (start 121 110.5) (end 124.4 107.1) (width 0.25) (layer "F.Cu") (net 72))
 (segment (start 78.665 89.5) (end 79.31 88.855) (width 0.25) (layer "F.Cu") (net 75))
 (segment (start 79.31 88.855) (end 80.865 88.855) (width 0.25) (layer "F.Cu") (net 75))
 (segment (start 80.865 88.855) (end 81.51 89.5) (width 0.25) (layer "F.Cu") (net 75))
 (segment (start 84.51 93.5) (end 87.025 93.5) (width 0.25) (layer "F.Cu") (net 29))
 (segment (start 79.165 108.825) (end 78.49 109.5) (width 0.25) (layer "F.Cu") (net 73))
 (segment (start 79.165 107) (end 79.165 108.825) (width 0.25) (layer "F.Cu") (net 73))
 (segment (start 112.87 99.88) (end 110.25 99.88) (width 0.25) (layer "F.Cu") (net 51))
 (segment (start 112.99 100) (end 112.87 99.88) (width 0.25) (layer "F.Cu") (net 51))
 (segment (start 112.99 98) (end 112.38 98.61) (width 0.25) (layer "F.Cu") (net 52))
 (segment (start 112.38 98.61) (end 110.25 98.61) (width 0.25) (layer "F.Cu") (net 52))
 (segment (start 107.985 98.435) (end 107.985 95.495) (width 0.25) (layer "F.Cu") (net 40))
 (segment (start 107.985 95.495) (end 105.49 93) (width 0.25) (layer "F.Cu") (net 40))
 (segment (start 105.94 97.36) (end 105.94 97.94) (width 0.25) (layer "F.Cu") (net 40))
 (segment (start 106.435 98.435) (end 107.985 98.435) (width 0.25) (layer "F.Cu") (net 40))
 (segment (start 105.94 97.94) (end 106.435 98.435) (width 0.25) (layer "F.Cu") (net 40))
 (segment (start 101.55 93.65) (end 101.55 96.09) (width 0.25) (layer "F.Cu") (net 35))
 (segment (start 101.55 96.09) (end 100.86 96.78) (width 0.25) (layer "F.Cu") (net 35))
 (segment (start 100.86 96.78) (end 100.86 97.36) (width 0.25) (layer "F.Cu") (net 35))
 (segment (start 99.45 93.65) (end 99.45 97.22) (width 0.25) (layer "F.Cu") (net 38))
 (segment (start 99.45 97.22) (end 99.59 97.36) (width 0.25) (layer "F.Cu") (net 38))
 (segment (start 97.05 97.36) (end 97.05 90.56) (width 0.25) (layer "F.Cu") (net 57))
 (segment (start 97.05 90.56) (end 96.99 90.5) (width 0.25) (layer "F.Cu") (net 57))
 (segment (start 83.49 93.5) (end 83.25 93.5) (width 0.25) (layer "F.Cu") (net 28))
 (segment (start 83.25 93.5) (end 81.75 95) (width 0.25) (layer "F.Cu") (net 28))
 (segment (start 80.49 89.5) (end 80.49 90.5) (width 0.25) (layer "F.Cu") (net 28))
 (segment (start 80.49 90.5) (end 83.49 93.5) (width 0.25) (layer "F.Cu") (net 28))
 (segment (start 77.99 92.5) (end 77.99 92.74) (width 0.25) (layer "F.Cu") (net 77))
 (segment (start 77.99 92.74) (end 80.25 95) (width 0.25) (layer "F.Cu") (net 77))
 (segment (start 114.01 100) (end 122.5 100) (width 0.25) (layer "F.Cu") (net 31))
 (segment (start 114.01 98) (end 114.51 97.5) (width 0.25) (layer "F.Cu") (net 32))
 (segment (start 114.51 97.5) (end 122.5 97.5) (width 0.25) (layer "F.Cu") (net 32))
 (segment (start 106.51 93) (end 108.51 95) (width 0.25) (layer "F.Cu") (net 33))
 (segment (start 108.51 95) (end 122.5 95) (width 0.25) (layer "F.Cu") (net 33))
 (segment (start 98.01 90.5) (end 120.5 90.5) (width 0.25) (layer "F.Cu") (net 34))
 (segment (start 120.5 90.5) (end 122.5 92.5) (width 0.25) (layer "F.Cu") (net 34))
 (segment (start 79.51 109.5) (end 81.5 111.49) (width 0.25) (layer "F.Cu") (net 74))
 (segment (start 81.5 111.49) (end 81.5 114) (width 0.25) (layer "F.Cu") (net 74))
 (segment (start 84.655 86.345) (end 84.655 84.425) (width 0.25) (layer "F.Cu") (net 1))
 (segment (start 82.95 107.03) (end 82.95 115.45) (width 0.4) (layer "F.Cu") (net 1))
 (segment (start 84.38 84.05) (end 84.33 84.1) (width 0.25) (layer "F.Cu") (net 1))
 (segment (start 109.1 101.3) (end 109.1 97.425) (width 0.4) (layer "F.Cu") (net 1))
 (segment (start 123.55 96.25) (end 123.875 95.925) (width 0.4) (layer "F.Cu") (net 1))
 (segment (start 103 107.4) (end 103 108.8) (width 0.4) (layer "F.Cu") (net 1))
 (segment (start 78.375 102.5) (end 79.25 102.5) (width 0.25) (layer "F.Cu") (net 1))
 (segment (start 104.4 110.42) (end 104.4 108.8) (width 0.4) (layer "F.Cu") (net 1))
 (segment (start 80.432959 86.901) (end 84.099 86.901) (width 0.25) (layer "F.Cu") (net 1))
 (segment (start 101.6 108.8) (end 101.6 107.4) (width 0.4) (layer "F.Cu") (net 1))
 (segment (start 104.4 107.4) (end 104.4 106) (width 0.4) (layer "F.Cu") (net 1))
 (segment (start 78.025 89.308959) (end 80.432959 86.901) (width 0.25) (layer "F.Cu") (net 1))
 (segment (start 109.1 97.425) (end 110.275 96.25) (width 0.4) (layer "F.Cu") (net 1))
 (segment (start 85 104.02) (end 83.64 104.02) (width 0.4) (layer "F.Cu") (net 1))
 (segment (start 78.025 91) (end 78.025 91.515) (width 0.25) (layer "F.Cu") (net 1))
 (segment (start 102.175 93) (end 101.55 93) (width 0.4) (layer "F.Cu") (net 1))
 (segment (start 92.37 115.5) (end 92.75 115.12) (width 0.4) (layer "F.Cu") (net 1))
 (segment (start 103 106) (end 103 107.4) (width 0.4) (layer "F.Cu") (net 1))
 (segment (start 101.55 93) (end 103.43 93) (width 0.25) (layer "F.Cu") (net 1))
 (segment (start 82.95 115.45) (end 83 115.5) (width 0.4) (layer "F.Cu") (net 1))
 (segment (start 123.142767 93.75) (end 108.336604 93.75) (width 0.4) (layer "F.Cu") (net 1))
 (segment (start 109.1 115.12) (end 104.4 110.42) (width 0.4) (layer "F.Cu") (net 1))
 (segment (start 120.26 115.12) (end 121 114.38) (width 0.4) (layer "F.Cu") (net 1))
 (segment (start 81.75 103.45) (end 82.98 104.68) (width 0.4) (layer "F.Cu") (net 1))
 (segment (start 78.025 89.5) (end 78.025 89.308959) (width 0.25) (layer "F.Cu") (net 1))
 (segment (start 123.875 94.482233) (end 123.142767 93.75) (width 0.4) (layer "F.Cu") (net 1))
 (segment (start 110.25 115.12) (end 120.26 115.12) (width 0.4) (layer "F.Cu") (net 1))
 (segment (start 104.4 108.8) (end 104.4 107.4) (width 0.4) (layer "F.Cu") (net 1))
 (segment (start 80.725 101.225) (end 80 100.5) (width 0.4) (layer "F.Cu") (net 1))
 (segment (start 78.025 89.5) (end 78.025 91) (width 0.25) (layer "F.Cu") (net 1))
 (segment (start 78.025 91.515) (end 79.01 92.5) (width 0.25) (layer "F.Cu") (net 1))
 (segment (start 80.725 102.425) (end 80.725 101.225) (width 0.4) (layer "F.Cu") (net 1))
 (segment (start 101.6 107.4) (end 101.6 106) (width 0.4) (layer "F.Cu") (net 1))
 (segment (start 78.02 102.145) (end 78.375 102.5) (width 0.25) (layer "F.Cu") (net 1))
 (segment (start 78.02 99) (end 78.02 100.5) (width 0.25) (layer "F.Cu") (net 1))
 (segment (start 95.28 115.12) (end 101.6 108.8) (width 0.4) (layer "F.Cu") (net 1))
 (segment (start 103 108.8) (end 104.4 108.8) (width 0.4) (layer "F.Cu") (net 1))
 (segment (start 82.98 104.68) (end 82.98 107) (width 0.4) (layer "F.Cu") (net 1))
 (segment (start 79.45 92.5) (end 81.25 94.3) (width 0.25) (layer "F.Cu") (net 1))
 (segment (start 80 100.5) (end 78.02 100.5) (width 0.4) (layer "F.Cu") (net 1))
 (segment (start 78.02 99) (end 78.02 97) (width 0.25) (layer "F.Cu") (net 1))
 (segment (start 108.336604 93.75) (end 106.836604 92.25) (width 0.4) (layer "F.Cu") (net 1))
 (segment (start 83.64 104.02) (end 82.98 104.68) (width 0.4) (layer "F.Cu") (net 1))
 (segment (start 103.43 93) (end 107.21 96.78) (width 0.25) (layer "F.Cu") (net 1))
 (segment (start 81.75 103.45) (end 80.725 102.425) (width 0.4) (layer "F.Cu") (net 1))
 (segment (start 82.98 107) (end 82.95 107.03) (width 0.4) (layer "F.Cu") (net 1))
 (segment (start 84.655 84.425) (end 84.33 84.1) (width 0.25) (layer "F.Cu") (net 1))
 (segment (start 78.02 100.5) (end 78.02 102.145) (width 0.25) (layer "F.Cu") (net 1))
 (segment (start 81.25 94.3) (end 81.25 95) (width 0.25) (layer "F.Cu") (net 1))
 (segment (start 110.25 115.12) (end 109.1 115.12) (width 0.4) (layer "F.Cu") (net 1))
 (segment (start 107.21 96.78) (end 107.21 97.36) (width 0.25) (layer "F.Cu") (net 1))
 (segment (start 78.02 97) (end 77.395 96.375) (width 0.25) (layer "F.Cu") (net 1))
 (segment (start 84.099 86.901) (end 84.655 86.345) (width 0.25) (layer "F.Cu") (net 1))
 (segment (start 92.75 115.12) (end 95.28 115.12) (width 0.4) (layer "F.Cu") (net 1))
 (segment (start 123.875 95.925) (end 123.875 94.482233) (width 0.4) (layer "F.Cu") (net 1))
 (segment (start 85.58 84.05) (end 84.38 84.05) (width 0.25) (layer "F.Cu") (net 1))
 (segment (start 110.275 96.25) (end 123.55 96.25) (width 0.4) (layer "F.Cu") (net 1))
 (segment (start 79.01 92.5) (end 79.45 92.5) (width 0.25) (layer "F.Cu") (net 1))
 (segment (start 77.395 91.63) (end 78.025 91) (width 0.25) (layer "F.Cu") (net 1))
 (segment (start 101.6 106) (end 103 106) (width 0.4) (layer "F.Cu") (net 1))
 (segment (start 77.395 96.375) (end 77.395 91.63) (width 0.25) (layer "F.Cu") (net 1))
 (segment (start 104.4 106) (end 109.1 101.3) (width 0.4) (layer "F.Cu") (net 1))
 (segment (start 106.836604 92.25) (end 102.925 92.25) (width 0.4) (layer "F.Cu") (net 1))
 (segment (start 83 115.5) (end 92.37 115.5) (width 0.4) (layer "F.Cu") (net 1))
 (segment (start 102.925 92.25) (end 102.175 93) (width 0.4) (layer "F.Cu") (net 1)))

